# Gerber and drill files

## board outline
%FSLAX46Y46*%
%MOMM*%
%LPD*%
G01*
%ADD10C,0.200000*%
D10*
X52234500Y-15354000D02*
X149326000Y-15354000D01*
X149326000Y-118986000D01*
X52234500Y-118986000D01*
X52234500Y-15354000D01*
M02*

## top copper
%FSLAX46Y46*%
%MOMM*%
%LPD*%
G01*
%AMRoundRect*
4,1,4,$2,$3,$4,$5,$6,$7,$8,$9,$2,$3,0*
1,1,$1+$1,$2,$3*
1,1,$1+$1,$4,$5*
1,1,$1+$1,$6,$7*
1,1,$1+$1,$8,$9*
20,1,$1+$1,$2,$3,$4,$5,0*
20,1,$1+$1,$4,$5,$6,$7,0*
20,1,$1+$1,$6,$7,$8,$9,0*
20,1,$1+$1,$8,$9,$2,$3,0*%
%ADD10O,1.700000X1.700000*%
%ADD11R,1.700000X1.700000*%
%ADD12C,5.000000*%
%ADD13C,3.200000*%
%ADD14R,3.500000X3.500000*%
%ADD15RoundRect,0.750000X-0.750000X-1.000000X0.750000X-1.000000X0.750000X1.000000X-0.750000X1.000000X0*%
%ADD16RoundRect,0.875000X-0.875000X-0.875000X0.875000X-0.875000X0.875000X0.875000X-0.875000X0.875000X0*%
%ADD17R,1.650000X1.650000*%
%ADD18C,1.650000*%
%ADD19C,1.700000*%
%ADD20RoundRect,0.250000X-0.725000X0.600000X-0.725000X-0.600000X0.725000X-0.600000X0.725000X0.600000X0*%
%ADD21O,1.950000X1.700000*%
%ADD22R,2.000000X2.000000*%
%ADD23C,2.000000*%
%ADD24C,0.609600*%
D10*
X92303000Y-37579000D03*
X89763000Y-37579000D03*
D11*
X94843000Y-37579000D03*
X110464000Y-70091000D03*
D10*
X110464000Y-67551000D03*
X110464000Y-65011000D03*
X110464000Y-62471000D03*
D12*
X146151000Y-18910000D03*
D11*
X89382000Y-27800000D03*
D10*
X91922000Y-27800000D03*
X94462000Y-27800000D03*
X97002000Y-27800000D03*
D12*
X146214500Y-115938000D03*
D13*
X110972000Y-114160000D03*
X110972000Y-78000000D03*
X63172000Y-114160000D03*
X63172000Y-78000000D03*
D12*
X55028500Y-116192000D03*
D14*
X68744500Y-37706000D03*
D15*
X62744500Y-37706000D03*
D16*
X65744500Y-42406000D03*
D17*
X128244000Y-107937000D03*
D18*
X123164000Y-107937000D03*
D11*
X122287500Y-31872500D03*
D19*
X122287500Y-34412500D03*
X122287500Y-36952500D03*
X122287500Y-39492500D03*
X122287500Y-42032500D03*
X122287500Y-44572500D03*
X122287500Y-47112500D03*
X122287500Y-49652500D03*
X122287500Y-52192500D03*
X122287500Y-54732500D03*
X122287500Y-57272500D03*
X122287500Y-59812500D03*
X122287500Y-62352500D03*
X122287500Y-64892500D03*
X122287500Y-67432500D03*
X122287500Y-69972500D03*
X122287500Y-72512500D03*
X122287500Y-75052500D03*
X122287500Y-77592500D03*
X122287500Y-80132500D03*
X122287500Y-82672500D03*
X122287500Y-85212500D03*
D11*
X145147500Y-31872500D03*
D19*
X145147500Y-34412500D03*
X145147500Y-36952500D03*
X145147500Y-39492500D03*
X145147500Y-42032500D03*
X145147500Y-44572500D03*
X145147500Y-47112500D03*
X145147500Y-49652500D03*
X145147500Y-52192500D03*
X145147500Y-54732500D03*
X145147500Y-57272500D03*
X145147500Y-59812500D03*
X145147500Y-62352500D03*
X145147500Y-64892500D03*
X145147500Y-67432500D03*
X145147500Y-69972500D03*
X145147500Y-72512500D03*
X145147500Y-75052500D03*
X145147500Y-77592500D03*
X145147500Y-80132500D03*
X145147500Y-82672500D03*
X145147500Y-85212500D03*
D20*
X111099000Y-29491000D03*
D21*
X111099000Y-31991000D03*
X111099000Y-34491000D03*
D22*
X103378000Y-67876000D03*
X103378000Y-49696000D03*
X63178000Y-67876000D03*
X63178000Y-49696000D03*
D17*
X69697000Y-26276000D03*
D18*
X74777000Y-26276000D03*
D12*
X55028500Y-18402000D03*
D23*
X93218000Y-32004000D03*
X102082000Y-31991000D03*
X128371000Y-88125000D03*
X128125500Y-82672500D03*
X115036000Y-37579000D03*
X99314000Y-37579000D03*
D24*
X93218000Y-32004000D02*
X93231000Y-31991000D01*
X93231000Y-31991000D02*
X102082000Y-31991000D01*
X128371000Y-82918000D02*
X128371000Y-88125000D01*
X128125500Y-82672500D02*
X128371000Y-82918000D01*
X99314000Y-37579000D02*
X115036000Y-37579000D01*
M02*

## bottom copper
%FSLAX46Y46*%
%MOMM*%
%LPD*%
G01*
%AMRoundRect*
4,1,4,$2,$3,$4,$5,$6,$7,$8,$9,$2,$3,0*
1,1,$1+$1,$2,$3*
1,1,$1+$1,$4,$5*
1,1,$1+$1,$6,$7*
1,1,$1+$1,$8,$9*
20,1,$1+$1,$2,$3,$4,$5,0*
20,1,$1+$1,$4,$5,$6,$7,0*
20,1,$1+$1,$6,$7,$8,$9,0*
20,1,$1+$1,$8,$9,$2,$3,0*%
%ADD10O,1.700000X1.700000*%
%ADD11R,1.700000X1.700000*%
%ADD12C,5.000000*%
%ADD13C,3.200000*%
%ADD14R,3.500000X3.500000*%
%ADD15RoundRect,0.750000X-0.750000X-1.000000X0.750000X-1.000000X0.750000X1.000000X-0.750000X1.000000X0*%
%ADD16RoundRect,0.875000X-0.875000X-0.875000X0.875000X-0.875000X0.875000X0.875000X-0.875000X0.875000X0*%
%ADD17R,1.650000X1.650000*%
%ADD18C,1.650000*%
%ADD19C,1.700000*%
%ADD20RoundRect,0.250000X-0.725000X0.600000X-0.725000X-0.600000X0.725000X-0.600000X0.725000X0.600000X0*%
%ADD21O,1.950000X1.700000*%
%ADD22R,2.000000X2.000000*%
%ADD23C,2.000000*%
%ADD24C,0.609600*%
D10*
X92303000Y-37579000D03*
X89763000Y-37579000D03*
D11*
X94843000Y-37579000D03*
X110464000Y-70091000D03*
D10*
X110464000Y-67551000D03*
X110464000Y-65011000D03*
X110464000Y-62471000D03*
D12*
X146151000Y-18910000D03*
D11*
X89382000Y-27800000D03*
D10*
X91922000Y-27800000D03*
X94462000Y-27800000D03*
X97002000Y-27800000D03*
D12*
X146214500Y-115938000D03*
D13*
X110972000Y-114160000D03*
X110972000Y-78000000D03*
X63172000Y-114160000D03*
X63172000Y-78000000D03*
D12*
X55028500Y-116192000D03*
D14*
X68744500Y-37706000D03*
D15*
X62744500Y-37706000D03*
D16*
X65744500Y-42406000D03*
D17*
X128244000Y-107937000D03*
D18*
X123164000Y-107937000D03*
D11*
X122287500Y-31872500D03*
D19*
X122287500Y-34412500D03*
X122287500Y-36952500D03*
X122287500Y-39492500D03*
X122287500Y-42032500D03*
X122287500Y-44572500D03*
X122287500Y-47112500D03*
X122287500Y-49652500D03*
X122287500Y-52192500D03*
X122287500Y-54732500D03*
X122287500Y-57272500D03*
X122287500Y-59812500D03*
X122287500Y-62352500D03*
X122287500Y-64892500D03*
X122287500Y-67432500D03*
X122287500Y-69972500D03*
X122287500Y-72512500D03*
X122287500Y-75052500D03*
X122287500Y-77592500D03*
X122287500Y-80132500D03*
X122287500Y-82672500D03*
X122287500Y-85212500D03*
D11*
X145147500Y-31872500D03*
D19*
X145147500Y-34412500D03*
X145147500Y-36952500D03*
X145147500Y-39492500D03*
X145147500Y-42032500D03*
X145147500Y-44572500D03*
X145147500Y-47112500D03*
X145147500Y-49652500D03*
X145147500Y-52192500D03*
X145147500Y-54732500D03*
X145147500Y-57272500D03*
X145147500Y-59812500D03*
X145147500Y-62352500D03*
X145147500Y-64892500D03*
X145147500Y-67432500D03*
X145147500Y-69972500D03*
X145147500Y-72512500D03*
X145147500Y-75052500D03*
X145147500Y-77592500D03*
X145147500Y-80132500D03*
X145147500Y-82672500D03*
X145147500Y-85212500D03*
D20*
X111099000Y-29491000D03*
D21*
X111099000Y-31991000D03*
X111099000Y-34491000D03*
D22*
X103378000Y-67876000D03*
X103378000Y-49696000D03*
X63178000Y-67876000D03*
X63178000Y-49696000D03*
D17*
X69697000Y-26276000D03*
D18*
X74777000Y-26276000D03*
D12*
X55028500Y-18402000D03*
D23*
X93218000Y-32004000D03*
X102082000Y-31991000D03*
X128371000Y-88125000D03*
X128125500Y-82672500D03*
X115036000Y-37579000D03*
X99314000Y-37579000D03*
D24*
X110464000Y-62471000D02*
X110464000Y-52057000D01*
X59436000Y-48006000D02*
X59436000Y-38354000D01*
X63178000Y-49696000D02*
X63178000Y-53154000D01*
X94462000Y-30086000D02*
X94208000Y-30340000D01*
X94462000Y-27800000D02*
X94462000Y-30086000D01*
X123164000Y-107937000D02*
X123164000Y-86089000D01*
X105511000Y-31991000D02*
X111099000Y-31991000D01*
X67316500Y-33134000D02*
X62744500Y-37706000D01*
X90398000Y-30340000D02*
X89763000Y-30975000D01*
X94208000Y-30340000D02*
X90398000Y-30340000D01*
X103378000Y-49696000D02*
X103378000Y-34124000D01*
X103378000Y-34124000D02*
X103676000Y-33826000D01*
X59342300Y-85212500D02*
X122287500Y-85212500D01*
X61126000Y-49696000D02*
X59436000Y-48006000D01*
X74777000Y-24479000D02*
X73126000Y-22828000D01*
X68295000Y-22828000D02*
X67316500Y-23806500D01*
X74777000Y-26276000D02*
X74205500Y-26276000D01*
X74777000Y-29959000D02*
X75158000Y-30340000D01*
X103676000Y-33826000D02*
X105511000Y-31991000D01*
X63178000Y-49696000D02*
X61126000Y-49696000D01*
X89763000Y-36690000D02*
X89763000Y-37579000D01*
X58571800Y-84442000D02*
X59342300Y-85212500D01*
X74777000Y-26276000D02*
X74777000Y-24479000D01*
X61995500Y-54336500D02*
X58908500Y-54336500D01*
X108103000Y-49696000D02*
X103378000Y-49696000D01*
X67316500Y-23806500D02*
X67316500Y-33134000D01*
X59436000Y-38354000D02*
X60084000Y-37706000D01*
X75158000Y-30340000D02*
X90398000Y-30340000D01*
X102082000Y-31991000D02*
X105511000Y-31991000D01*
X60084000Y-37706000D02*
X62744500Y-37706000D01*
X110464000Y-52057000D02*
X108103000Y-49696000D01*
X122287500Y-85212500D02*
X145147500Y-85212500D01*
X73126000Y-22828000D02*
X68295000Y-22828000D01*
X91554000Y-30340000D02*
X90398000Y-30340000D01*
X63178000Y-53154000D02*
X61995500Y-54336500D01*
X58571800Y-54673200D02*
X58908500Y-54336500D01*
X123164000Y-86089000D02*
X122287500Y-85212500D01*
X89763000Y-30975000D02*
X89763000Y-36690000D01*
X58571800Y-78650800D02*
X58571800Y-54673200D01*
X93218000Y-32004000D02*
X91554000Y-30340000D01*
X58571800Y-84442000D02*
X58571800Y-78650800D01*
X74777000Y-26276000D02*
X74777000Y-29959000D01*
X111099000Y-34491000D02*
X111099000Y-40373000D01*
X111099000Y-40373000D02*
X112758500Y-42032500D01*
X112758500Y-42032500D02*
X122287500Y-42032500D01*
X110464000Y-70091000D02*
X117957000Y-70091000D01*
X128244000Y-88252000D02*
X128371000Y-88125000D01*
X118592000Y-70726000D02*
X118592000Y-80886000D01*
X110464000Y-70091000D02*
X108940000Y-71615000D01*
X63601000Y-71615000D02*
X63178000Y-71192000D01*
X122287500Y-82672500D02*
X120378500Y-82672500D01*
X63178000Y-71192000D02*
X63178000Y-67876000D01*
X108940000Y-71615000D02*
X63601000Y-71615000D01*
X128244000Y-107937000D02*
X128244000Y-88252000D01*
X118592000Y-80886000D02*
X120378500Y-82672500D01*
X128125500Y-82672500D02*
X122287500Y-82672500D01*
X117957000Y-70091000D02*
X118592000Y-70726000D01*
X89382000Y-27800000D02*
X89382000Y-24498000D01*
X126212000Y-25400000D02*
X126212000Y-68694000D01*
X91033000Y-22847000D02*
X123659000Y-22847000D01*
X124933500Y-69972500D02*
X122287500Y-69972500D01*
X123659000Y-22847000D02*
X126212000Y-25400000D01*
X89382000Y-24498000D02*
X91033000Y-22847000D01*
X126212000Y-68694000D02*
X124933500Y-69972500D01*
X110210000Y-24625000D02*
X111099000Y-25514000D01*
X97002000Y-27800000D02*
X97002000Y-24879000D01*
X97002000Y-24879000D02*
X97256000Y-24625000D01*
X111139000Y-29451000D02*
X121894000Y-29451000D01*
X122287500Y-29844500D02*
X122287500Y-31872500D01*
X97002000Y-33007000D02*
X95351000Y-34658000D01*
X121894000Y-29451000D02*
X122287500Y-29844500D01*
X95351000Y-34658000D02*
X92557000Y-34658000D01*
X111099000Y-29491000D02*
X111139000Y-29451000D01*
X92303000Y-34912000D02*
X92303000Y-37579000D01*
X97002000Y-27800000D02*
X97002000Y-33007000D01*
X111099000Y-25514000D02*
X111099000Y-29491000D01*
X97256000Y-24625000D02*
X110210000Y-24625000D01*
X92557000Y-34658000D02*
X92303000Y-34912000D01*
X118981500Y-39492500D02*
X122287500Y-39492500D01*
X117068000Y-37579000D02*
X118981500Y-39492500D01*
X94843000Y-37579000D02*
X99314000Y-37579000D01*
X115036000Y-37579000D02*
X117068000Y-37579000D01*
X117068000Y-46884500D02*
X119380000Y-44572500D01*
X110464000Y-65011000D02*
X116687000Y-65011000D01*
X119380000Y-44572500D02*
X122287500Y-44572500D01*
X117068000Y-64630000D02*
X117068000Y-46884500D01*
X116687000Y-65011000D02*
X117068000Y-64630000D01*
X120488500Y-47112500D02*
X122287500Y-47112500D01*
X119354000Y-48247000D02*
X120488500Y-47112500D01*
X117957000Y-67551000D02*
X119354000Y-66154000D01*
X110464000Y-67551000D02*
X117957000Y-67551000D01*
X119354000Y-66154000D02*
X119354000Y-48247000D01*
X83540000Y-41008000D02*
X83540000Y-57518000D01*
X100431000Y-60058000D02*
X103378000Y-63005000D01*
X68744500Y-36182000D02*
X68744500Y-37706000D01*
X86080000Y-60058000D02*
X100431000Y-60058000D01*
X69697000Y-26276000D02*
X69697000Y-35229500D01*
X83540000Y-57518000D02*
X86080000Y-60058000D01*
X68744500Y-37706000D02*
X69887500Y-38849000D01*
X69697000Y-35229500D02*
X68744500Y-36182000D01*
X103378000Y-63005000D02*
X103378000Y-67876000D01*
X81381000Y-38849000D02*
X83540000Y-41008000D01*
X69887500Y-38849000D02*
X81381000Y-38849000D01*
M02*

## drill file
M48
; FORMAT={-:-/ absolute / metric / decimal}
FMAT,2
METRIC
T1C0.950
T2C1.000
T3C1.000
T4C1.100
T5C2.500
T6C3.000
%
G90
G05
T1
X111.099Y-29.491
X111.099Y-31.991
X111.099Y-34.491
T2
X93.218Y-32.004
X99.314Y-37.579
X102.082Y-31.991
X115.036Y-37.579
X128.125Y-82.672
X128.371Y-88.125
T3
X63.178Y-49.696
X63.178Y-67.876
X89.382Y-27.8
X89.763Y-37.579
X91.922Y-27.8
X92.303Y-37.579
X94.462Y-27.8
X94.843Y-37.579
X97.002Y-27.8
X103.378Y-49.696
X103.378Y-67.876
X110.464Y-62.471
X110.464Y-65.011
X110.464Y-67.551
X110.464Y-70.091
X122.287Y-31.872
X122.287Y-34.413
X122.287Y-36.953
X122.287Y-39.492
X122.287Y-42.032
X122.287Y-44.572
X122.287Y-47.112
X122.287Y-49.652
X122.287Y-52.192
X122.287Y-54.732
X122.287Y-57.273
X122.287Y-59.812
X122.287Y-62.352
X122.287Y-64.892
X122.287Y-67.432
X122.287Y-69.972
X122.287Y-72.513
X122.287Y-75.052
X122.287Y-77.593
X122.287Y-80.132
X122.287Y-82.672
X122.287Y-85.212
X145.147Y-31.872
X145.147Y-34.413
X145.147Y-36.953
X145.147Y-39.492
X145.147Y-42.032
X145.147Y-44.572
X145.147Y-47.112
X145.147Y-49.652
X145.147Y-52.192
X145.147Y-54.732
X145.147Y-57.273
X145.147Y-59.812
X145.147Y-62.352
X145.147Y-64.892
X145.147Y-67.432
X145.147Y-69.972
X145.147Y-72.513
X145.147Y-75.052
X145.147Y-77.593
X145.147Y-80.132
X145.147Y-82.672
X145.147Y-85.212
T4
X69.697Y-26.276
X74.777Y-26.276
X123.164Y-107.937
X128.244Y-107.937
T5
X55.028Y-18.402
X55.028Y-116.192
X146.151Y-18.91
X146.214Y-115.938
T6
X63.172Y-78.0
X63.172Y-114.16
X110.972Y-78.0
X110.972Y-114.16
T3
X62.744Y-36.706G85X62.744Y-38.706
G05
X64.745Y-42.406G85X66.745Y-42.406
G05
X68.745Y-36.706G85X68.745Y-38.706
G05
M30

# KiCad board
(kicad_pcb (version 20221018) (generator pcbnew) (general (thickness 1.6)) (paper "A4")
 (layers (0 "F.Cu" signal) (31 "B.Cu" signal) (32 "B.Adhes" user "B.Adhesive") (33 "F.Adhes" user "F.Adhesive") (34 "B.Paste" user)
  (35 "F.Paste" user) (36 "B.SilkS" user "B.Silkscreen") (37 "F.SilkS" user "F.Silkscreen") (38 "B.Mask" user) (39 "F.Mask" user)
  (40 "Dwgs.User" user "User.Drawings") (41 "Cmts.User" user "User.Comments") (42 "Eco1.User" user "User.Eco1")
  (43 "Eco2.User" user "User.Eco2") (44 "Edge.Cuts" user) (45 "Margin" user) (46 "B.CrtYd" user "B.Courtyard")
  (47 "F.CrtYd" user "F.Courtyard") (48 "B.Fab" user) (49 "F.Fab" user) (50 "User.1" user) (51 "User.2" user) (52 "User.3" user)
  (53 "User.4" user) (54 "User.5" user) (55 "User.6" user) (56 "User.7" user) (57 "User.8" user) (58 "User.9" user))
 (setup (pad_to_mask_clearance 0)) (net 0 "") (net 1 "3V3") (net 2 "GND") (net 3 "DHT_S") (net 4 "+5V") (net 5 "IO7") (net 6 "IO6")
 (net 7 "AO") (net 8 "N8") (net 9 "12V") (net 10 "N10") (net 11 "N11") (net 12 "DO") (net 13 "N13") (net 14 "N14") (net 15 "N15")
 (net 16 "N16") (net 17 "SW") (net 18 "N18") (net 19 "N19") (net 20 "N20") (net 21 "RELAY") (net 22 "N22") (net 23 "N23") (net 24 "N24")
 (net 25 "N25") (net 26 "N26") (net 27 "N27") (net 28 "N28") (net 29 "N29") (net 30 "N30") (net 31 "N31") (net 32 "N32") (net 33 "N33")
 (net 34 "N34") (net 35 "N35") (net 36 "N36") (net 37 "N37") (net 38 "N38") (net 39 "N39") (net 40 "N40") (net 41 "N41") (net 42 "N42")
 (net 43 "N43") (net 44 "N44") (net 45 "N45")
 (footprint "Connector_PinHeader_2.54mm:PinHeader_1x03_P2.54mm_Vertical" (layer "F.Cu") (at 94.843 37.579 -90)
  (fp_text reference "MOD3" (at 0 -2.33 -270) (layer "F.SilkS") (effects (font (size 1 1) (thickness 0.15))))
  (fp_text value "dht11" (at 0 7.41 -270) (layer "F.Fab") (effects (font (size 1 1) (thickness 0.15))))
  (pad "+" thru_hole oval (at 0 2.54 270) (size 1.7 1.7) (drill 1) (layers "*.Cu" "*.Mask") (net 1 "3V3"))
  (pad "-" thru_hole oval (at 0 5.08 270) (size 1.7 1.7) (drill 1) (layers "*.Cu" "*.Mask") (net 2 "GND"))
  (pad "S" thru_hole rect (at 0 0 270) (size 1.7 1.7) (drill 1) (layers "*.Cu" "*.Mask") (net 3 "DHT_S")))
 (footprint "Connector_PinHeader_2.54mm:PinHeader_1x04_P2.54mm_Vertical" (layer "F.Cu") (at 110.464 70.091 180)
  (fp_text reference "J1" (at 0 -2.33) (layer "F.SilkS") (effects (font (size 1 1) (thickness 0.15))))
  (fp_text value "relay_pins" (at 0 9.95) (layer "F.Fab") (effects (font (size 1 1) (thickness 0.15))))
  (pad "1" thru_hole rect (at 0 0 180) (size 1.7 1.7) (drill 1) (layers "*.Cu" "*.Mask") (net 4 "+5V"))
  (pad "2" thru_hole oval (at 0 2.54 180) (size 1.7 1.7) (drill 1) (layers "*.Cu" "*.Mask") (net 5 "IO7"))
  (pad "3" thru_hole oval (at 0 5.08 180) (size 1.7 1.7) (drill 1) (layers "*.Cu" "*.Mask") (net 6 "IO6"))
  (pad "4" thru_hole oval (at 0 7.62 180) (size 1.7 1.7) (drill 1) (layers "*.Cu" "*.Mask") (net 2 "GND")))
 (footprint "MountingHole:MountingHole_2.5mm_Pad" (layer "F.Cu") (at 146.151 18.91)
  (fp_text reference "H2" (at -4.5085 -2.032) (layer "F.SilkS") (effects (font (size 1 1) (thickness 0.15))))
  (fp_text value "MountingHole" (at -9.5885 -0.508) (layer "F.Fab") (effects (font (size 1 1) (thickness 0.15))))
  (pad "1" thru_hole circle (at 0 0) (size 5 5) (drill 2.5) (layers "*.Cu" "*.Mask")))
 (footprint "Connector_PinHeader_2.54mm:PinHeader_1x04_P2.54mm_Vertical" (layer "F.Cu") (at 89.382 27.8 90)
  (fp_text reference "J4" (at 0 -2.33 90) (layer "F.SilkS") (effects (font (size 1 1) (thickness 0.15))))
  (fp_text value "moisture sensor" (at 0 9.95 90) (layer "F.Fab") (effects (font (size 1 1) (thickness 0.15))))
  (pad "1" thru_hole rect (at 0 0 90) (size 1.7 1.7) (drill 1) (layers "*.Cu" "*.Mask") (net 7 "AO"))
  (pad "2" thru_hole oval (at 0 2.54 90) (size 1.7 1.7) (drill 1) (layers "*.Cu" "*.Mask") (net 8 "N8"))
  (pad "3" thru_hole oval (at 0 5.08 90) (size 1.7 1.7) (drill 1) (layers "*.Cu" "*.Mask") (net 2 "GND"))
  (pad "4" thru_hole oval (at 0 7.62 90) (size 1.7 1.7) (drill 1) (layers "*.Cu" "*.Mask") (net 1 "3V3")))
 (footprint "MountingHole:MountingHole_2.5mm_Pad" (layer "F.Cu") (at 146.2145 115.938)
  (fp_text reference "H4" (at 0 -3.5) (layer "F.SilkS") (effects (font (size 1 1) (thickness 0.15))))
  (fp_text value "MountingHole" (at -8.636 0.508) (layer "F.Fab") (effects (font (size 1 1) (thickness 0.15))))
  (pad "1" thru_hole circle (at 0 0) (size 5 5) (drill 2.5) (layers "*.Cu" "*.Mask")))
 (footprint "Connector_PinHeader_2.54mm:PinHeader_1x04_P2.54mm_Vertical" (layer "F.Cu") (at 110.972 114.16 180)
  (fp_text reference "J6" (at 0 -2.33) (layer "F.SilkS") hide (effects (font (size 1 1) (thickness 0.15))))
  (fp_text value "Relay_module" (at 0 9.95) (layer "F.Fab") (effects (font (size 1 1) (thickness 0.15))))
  (pad "" np_thru_hole circle (at 0 0 180) (size 3.2 3.2) (drill 3) (layers "F&B.Cu" "*.Mask"))
  (pad "" np_thru_hole circle (at 0 36.16 180) (size 3.2 3.2) (drill 3) (layers "F&B.Cu" "*.Mask"))
  (pad "" np_thru_hole circle (at 47.8 0 180) (size 3.2 3.2) (drill 3) (layers "F&B.Cu" "*.Mask"))
  (pad "" np_thru_hole circle (at 47.8 36.16 180) (size 3.2 3.2) (drill 3) (layers "F&B.Cu" "*.Mask")))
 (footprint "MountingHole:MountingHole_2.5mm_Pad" (layer "F.Cu") (at 55.0285 116.192)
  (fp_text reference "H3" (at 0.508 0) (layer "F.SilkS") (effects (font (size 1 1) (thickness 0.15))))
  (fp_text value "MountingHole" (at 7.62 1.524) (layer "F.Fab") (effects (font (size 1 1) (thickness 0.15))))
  (pad "1" thru_hole circle (at 0 0) (size 5 5) (drill 2.5) (layers "*.Cu" "*.Mask")))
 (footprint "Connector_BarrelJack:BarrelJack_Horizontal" (layer "F.Cu") (at 68.7445 37.706)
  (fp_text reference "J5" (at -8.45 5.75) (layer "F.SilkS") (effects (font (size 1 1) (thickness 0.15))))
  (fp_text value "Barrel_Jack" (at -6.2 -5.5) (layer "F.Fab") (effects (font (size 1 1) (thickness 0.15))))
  (pad "1" thru_hole rect (at 0 0) (size 3.5 3.5) (drill oval 1 3) (layers "*.Cu" "*.Mask") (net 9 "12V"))
  (pad "2" thru_hole roundrect (at -6 0) (size 3 3.5) (drill oval 1 3) (layers "*.Cu" "*.Mask") (roundrect_rratio 0.25) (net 2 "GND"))
  (pad "3" thru_hole roundrect (at -3 4.7) (size 3.5 3.5) (drill oval 3 1) (layers "*.Cu" "*.Mask") (roundrect_rratio 0.25)))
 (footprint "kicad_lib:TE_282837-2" (layer "F.Cu") (at 125.704 107.937 180)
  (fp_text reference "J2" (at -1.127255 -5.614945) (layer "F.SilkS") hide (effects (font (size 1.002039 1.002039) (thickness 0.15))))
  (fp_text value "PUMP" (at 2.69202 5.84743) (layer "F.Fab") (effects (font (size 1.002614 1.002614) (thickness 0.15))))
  (pad "1" thru_hole rect (at -2.54 0 180) (size 1.65 1.65) (drill 1.1) (layers "*.Cu" "*.Mask") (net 4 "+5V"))
  (pad "2" thru_hole circle (at 2.54 0 180) (size 1.65 1.65) (drill 1.1) (layers "*.Cu" "*.Mask") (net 2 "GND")))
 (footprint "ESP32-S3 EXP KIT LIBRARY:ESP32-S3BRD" (layer "F.Cu") (at 121.0175 96.6725)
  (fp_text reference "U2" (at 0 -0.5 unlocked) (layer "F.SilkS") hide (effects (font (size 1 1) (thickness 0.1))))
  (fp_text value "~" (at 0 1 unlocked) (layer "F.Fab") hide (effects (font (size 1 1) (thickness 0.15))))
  (pad "1_1" thru_hole rect (at 1.27 -64.8) (size 1.7 1.7) (drill 1) (layers "*.Cu" "*.Mask") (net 1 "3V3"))
  (pad "1_2" thru_hole circle (at 1.27 -62.26) (size 1.7 1.7) (drill 1) (layers "*.Cu" "*.Mask") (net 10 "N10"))
  (pad "1_3" thru_hole circle (at 1.27 -59.72) (size 1.7 1.7) (drill 1) (layers "*.Cu" "*.Mask") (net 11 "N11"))
  (pad "1_4" thru_hole circle (at 1.27 -57.18) (size 1.7 1.7) (drill 1) (layers "*.Cu" "*.Mask") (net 3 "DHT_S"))
  (pad "1_5" thru_hole circle (at 1.27 -54.64) (size 1.7 1.7) (drill 1) (layers "*.Cu" "*.Mask") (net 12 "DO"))
  (pad "1_6" thru_hole circle (at 1.27 -52.1) (size 1.7 1.7) (drill 1) (layers "*.Cu" "*.Mask") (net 6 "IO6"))
  (pad "1_7" thru_hole circle (at 1.27 -49.56) (size 1.7 1.7) (drill 1) (layers "*.Cu" "*.Mask") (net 5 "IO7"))
  (pad "1_8" thru_hole circle (at 1.27 -47.02) (size 1.7 1.7) (drill 1) (layers "*.Cu" "*.Mask") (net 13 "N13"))
  (pad "1_9" thru_hole circle (at 1.27 -44.48) (size 1.7 1.7) (drill 1) (layers "*.Cu" "*.Mask") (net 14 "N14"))
  (pad "1_10" thru_hole circle (at 1.27 -41.94) (size 1.7 1.7) (drill 1) (layers "*.Cu" "*.Mask") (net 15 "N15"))
  (pad "1_11" thru_hole circle (at 1.27 -39.4) (size 1.7 1.7) (drill 1) (layers "*.Cu" "*.Mask") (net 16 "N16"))
  (pad "1_12" thru_hole circle (at 1.27 -36.86) (size 1.7 1.7) (drill 1) (layers "*.Cu" "*.Mask") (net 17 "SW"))
  (pad "1_13" thru_hole circle (at 1.27 -34.32) (size 1.7 1.7) (drill 1) (layers "*.Cu" "*.Mask") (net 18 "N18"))
  (pad "1_14" thru_hole circle (at 1.27 -31.78) (size 1.7 1.7) (drill 1) (layers "*.Cu" "*.Mask") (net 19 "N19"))
  (pad "1_15" thru_hole circle (at 1.27 -29.24) (size 1.7 1.7) (drill 1) (layers "*.Cu" "*.Mask") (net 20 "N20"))
  (pad "1_16" thru_hole circle (at 1.27 -26.7) (size 1.7 1.7) (drill 1) (layers "*.Cu" "*.Mask") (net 7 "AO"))
  (pad "1_17" thru_hole circle (at 1.27 -24.16) (size 1.7 1.7) (drill 1) (layers "*.Cu" "*.Mask") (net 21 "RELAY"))
  (pad "1_18" thru_hole circle (at 1.27 -21.62) (size 1.7 1.7) (drill 1) (layers "*.Cu" "*.Mask") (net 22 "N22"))
  (pad "1_19" thru_hole circle (at 1.27 -19.08) (size 1.7 1.7) (drill 1) (layers "*.Cu" "*.Mask") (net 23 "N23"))
  (pad "1_20" thru_hole circle (at 1.27 -16.54) (size 1.7 1.7) (drill 1) (layers "*.Cu" "*.Mask") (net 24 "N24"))
  (pad "1_21" thru_hole circle (at 1.27 -14) (size 1.7 1.7) (drill 1) (layers "*.Cu" "*.Mask") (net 4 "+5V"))
  (pad "1_22" thru_hole circle (at 1.27 -11.46) (size 1.7 1.7) (drill 1) (layers "*.Cu" "*.Mask") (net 2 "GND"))
  (pad "2_1" thru_hole rect (at 24.13 -64.8) (size 1.7 1.7) (drill 1) (layers "*.Cu" "*.Mask") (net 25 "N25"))
  (pad "2_2" thru_hole circle (at 24.13 -62.26) (size 1.7 1.7) (drill 1) (layers "*.Cu" "*.Mask") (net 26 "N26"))
  (pad "2_3" thru_hole circle (at 24.13 -59.72) (size 1.7 1.7) (drill 1) (layers "*.Cu" "*.Mask") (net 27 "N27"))
  (pad "2_4" thru_hole circle (at 24.13 -57.18) (size 1.7 1.7) (drill 1) (layers "*.Cu" "*.Mask") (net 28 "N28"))
  (pad "2_5" thru_hole circle (at 24.13 -54.64) (size 1.7 1.7) (drill 1) (layers "*.Cu" "*.Mask") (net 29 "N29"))
  (pad "2_6" thru_hole circle (at 24.13 -52.1) (size 1.7 1.7) (drill 1) (layers "*.Cu" "*.Mask") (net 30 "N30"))
  (pad "2_7" thru_hole circle (at 24.13 -49.56) (size 1.7 1.7) (drill 1) (layers "*.Cu" "*.Mask") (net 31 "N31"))
  (pad "2_8" thru_hole circle (at 24.13 -47.02) (size 1.7 1.7) (drill 1) (layers "*.Cu" "*.Mask") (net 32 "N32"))
  (pad "2_9" thru_hole circle (at 24.13 -44.48) (size 1.7 1.7) (drill 1) (layers "*.Cu" "*.Mask") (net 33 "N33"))
  (pad "2_10" thru_hole circle (at 24.13 -41.94) (size 1.7 1.7) (drill 1) (layers "*.Cu" "*.Mask") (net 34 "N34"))
  (pad "2_11" thru_hole circle (at 24.13 -39.4) (size 1.7 1.7) (drill 1) (layers "*.Cu" "*.Mask") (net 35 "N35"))
  (pad "2_12" thru_hole circle (at 24.13 -36.86) (size 1.7 1.7) (drill 1) (layers "*.Cu" "*.Mask") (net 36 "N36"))
  (pad "2_13" thru_hole circle (at 24.13 -34.32) (size 1.7 1.7) (drill 1) (layers "*.Cu" "*.Mask") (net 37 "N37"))
  (pad "2_14" thru_hole circle (at 24.13 -31.78) (size 1.7 1.7) (drill 1) (layers "*.Cu" "*.Mask") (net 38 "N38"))
  (pad "2_15" thru_hole circle (at 24.13 -29.24) (size 1.7 1.7) (drill 1) (layers "*.Cu" "*.Mask") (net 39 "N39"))
  (pad "2_16" thru_hole circle (at 24.13 -26.7) (size 1.7 1.7) (drill 1) (layers "*.Cu" "*.Mask") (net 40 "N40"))
  (pad "2_17" thru_hole circle (at 24.13 -24.16) (size 1.7 1.7) (drill 1) (layers "*.Cu" "*.Mask") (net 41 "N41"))
  (pad "2_18" thru_hole circle (at 24.13 -21.62) (size 1.7 1.7) (drill 1) (layers "*.Cu" "*.Mask") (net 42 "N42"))
  (pad "2_19" thru_hole circle (at 24.13 -19.08) (size 1.7 1.7) (drill 1) (layers "*.Cu" "*.Mask") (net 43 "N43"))
  (pad "2_20" thru_hole circle (at 24.13 -16.54) (size 1.7 1.7) (drill 1) (layers "*.Cu" "*.Mask") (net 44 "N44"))
  (pad "2_21" thru_hole circle (at 24.13 -14) (size 1.7 1.7) (drill 1) (layers "*.Cu" "*.Mask") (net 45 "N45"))
  (pad "2_22" thru_hole circle (at 24.13 -11.46) (size 1.7 1.7) (drill 1) (layers "*.Cu" "*.Mask") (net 2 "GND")))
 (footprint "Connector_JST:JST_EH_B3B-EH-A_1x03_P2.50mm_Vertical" (layer "F.Cu") (at 111.099 29.491 -90)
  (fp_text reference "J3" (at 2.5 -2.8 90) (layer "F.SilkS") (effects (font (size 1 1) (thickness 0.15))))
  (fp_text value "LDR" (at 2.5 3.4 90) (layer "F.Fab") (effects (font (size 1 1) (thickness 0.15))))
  (pad "1" thru_hole roundrect (at 0 0 270) (size 1.7 1.95) (drill 0.95) (layers "*.Cu" "*.Mask") (roundrect_rratio 0.147059) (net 1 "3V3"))
  (pad "2" thru_hole oval (at 2.5 0 270) (size 1.7 1.95) (drill 0.95) (layers "*.Cu" "*.Mask") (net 2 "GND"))
  (pad "3" thru_hole oval (at 5 0 270) (size 1.7 1.95) (drill 0.95) (layers "*.Cu" "*.Mask") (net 12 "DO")))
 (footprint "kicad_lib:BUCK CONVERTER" (layer "F.Cu") (at 105.178 47.896 180)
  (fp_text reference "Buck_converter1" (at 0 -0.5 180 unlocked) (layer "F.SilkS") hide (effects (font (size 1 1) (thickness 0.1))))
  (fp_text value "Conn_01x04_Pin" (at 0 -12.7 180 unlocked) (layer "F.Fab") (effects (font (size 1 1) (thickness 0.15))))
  (pad "IN+" thru_hole rect (at 1.8 -19.98 180) (size 2 2) (drill 1) (layers "*.Cu" "*.Mask") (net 9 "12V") (thermal_bridge_angle 45))
  (pad "IN-" thru_hole rect (at 1.8 -1.8 180) (size 2 2) (drill 1) (layers "*.Cu" "B.Mask") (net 2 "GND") (thermal_bridge_angle 45))
  (pad "OUT+" thru_hole rect (at 42 -19.98 180) (size 2 2) (drill 1) (layers "*.Cu" "*.Mask") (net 4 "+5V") (thermal_bridge_angle 45))
  (pad "OUT-" thru_hole rect (at 42 -1.8 180) (size 2 2) (drill 1) (layers "*.Cu" "*.Mask") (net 2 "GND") (thermal_bridge_angle 45)))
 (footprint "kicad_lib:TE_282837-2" (layer "F.Cu") (at 72.237 26.276)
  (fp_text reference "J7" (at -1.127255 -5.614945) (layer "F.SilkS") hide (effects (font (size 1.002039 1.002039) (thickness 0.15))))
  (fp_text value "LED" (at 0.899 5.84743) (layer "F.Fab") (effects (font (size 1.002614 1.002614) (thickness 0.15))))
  (pad "1" thru_hole rect (at -2.54 0) (size 1.65 1.65) (drill 1.1) (layers "*.Cu" "*.Mask") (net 9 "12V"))
  (pad "2" thru_hole circle (at 2.54 0) (size 1.65 1.65) (drill 1.1) (layers "*.Cu" "*.Mask") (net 2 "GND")))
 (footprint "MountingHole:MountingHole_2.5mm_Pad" (layer "F.Cu") (at 55.0285 18.402)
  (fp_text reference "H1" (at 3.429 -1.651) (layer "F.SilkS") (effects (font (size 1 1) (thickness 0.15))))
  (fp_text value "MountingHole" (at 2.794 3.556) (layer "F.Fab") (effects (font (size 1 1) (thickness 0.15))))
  (pad "1" thru_hole circle (at 0 0) (size 5 5) (drill 2.5) (layers "*.Cu" "*.Mask")))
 (gr_rect (start 52.2345 15.354) (end 149.326 118.986) (stroke (width 0.2) (type default)) (fill none) (layer "Edge.Cuts"))
 (segment (start 93.218 32.004) (end 93.231 31.991) (width 0.6096) (layer "F.Cu") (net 2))
 (segment (start 93.231 31.991) (end 102.082 31.991) (width 0.6096) (layer "F.Cu") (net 2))
 (via (at 93.218 32.004) (size 2) (drill 1) (layers "F.Cu" "B.Cu") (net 2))
 (via (at 102.082 31.991) (size 2) (drill 1) (layers "F.Cu" "B.Cu") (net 2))
 (segment (start 110.464 62.471) (end 110.464 52.057) (width 0.6096) (layer "B.Cu") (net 2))
 (segment (start 59.436 48.006) (end 59.436 38.354) (width 0.6096) (layer "B.Cu") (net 2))
 (segment (start 63.178 49.696) (end 63.178 53.154) (width 0.6096) (layer "B.Cu") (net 2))
 (segment (start 94.462 30.086) (end 94.208 30.34) (width 0.6096) (layer "B.Cu") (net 2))
 (segment (start 94.462 27.8) (end 94.462 30.086) (width 0.6096) (layer "B.Cu") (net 2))
 (segment (start 123.164 107.937) (end 123.164 86.089) (width 0.6096) (layer "B.Cu") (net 2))
 (segment (start 105.511 31.991) (end 111.099 31.991) (width 0.6096) (layer "B.Cu") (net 2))
 (segment (start 67.3165 33.134) (end 62.7445 37.706) (width 0.6096) (layer "B.Cu") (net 2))
 (segment (start 90.398 30.34) (end 89.763 30.975) (width 0.6096) (layer "B.Cu") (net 2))
 (segment (start 94.208 30.34) (end 90.398 30.34) (width 0.6096) (layer "B.Cu") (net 2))
 (segment (start 103.378 49.696) (end 103.378 34.124) (width 0.6096) (layer "B.Cu") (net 2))
 (segment (start 103.378 34.124) (end 103.676 33.826) (width 0.6096) (layer "B.Cu") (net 2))
 (segment (start 59.3423 85.2125) (end 122.2875 85.2125) (width 0.6096) (layer "B.Cu") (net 2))
 (segment (start 61.126 49.696) (end 59.436 48.006) (width 0.6096) (layer "B.Cu") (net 2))
 (segment (start 74.777 24.479) (end 73.126 22.828) (width 0.6096) (layer "B.Cu") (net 2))
 (segment (start 68.295 22.828) (end 67.3165 23.8065) (width 0.6096) (layer "B.Cu") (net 2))
 (segment (start 74.777 26.276) (end 74.2055 26.276) (width 0.6096) (layer "B.Cu") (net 2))
 (segment (start 74.777 29.959) (end 75.158 30.34) (width 0.6096) (layer "B.Cu") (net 2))
 (segment (start 103.676 33.826) (end 105.511 31.991) (width 0.6096) (layer "B.Cu") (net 2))
 (segment (start 63.178 49.696) (end 61.126 49.696) (width 0.6096) (layer "B.Cu") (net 2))
 (segment (start 89.763 36.69) (end 89.763 37.579) (width 0.6096) (layer "B.Cu") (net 2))
 (segment (start 58.5718 84.442) (end 59.3423 85.2125) (width 0.6096) (layer "B.Cu") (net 2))
 (segment (start 74.777 26.276) (end 74.777 24.479) (width 0.6096) (layer "B.Cu") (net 2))
 (segment (start 61.9955 54.3365) (end 58.9085 54.3365) (width 0.6096) (layer "B.Cu") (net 2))
 (segment (start 108.103 49.696) (end 103.378 49.696) (width 0.6096) (layer "B.Cu") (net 2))
 (segment (start 67.3165 23.8065) (end 67.3165 33.134) (width 0.6096) (layer "B.Cu") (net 2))
 (segment (start 59.436 38.354) (end 60.084 37.706) (width 0.6096) (layer "B.Cu") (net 2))
 (segment (start 75.158 30.34) (end 90.398 30.34) (width 0.6096) (layer "B.Cu") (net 2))
 (segment (start 102.082 31.991) (end 105.511 31.991) (width 0.6096) (layer "B.Cu") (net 2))
 (segment (start 60.084 37.706) (end 62.7445 37.706) (width 0.6096) (layer "B.Cu") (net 2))
 (segment (start 110.464 52.057) (end 108.103 49.696) (width 0.6096) (layer "B.Cu") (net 2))
 (segment (start 122.2875 85.2125) (end 145.1475 85.2125) (width 0.6096) (layer "B.Cu") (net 2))
 (segment (start 73.126 22.828) (end 68.295 22.828) (width 0.6096) (layer "B.Cu") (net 2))
 (segment (start 91.554 30.34) (end 90.398 30.34) (width 0.6096) (layer "B.Cu") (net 2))
 (segment (start 63.178 53.154) (end 61.9955 54.3365) (width 0.6096) (layer "B.Cu") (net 2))
 (segment (start 58.5718 54.6732) (end 58.9085 54.3365) (width 0.6096) (layer "B.Cu") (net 2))
 (segment (start 123.164 86.089) (end 122.2875 85.2125) (width 0.6096) (layer "B.Cu") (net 2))
 (segment (start 89.763 30.975) (end 89.763 36.69) (width 0.6096) (layer "B.Cu") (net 2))
 (segment (start 58.5718 78.6508) (end 58.5718 54.6732) (width 0.6096) (layer "B.Cu") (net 2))
 (segment (start 93.218 32.004) (end 91.554 30.34) (width 0.6096) (layer "B.Cu") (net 2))
 (segment (start 58.5718 84.442) (end 58.5718 78.6508) (width 0.6096) (layer "B.Cu") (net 2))
 (segment (start 74.777 26.276) (end 74.777 29.959) (width 0.6096) (layer "B.Cu") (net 2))
 (segment (start 111.099 34.491) (end 111.099 40.373) (width 0.6096) (layer "B.Cu") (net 12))
 (segment (start 111.099 40.373) (end 112.7585 42.0325) (width 0.6096) (layer "B.Cu") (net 12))
 (segment (start 112.7585 42.0325) (end 122.2875 42.0325) (width 0.6096) (layer "B.Cu") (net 12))
 (segment (start 128.371 82.918) (end 128.371 88.125) (width 0.6096) (layer "F.Cu") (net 4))
 (segment (start 128.1255 82.6725) (end 128.371 82.918) (width 0.6096) (layer "F.Cu") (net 4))
 (via (at 128.371 88.125) (size 2) (drill 1) (layers "F.Cu" "B.Cu") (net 4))
 (via (at 128.1255 82.6725) (size 2) (drill 1) (layers "F.Cu" "B.Cu") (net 4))
 (segment (start 110.464 70.091) (end 117.957 70.091) (width 0.6096) (layer "B.Cu") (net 4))
 (segment (start 128.244 88.252) (end 128.371 88.125) (width 0.6096) (layer "B.Cu") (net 4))
 (segment (start 118.592 70.726) (end 118.592 80.886) (width 0.6096) (layer "B.Cu") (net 4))
 (segment (start 110.464 70.091) (end 108.94 71.615) (width 0.6096) (layer "B.Cu") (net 4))
 (segment (start 63.601 71.615) (end 63.178 71.192) (width 0.6096) (layer "B.Cu") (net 4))
 (segment (start 122.2875 82.6725) (end 120.3785 82.6725) (width 0.6096) (layer "B.Cu") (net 4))
 (segment (start 63.178 71.192) (end 63.178 67.876) (width 0.6096) (layer "B.Cu") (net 4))
 (segment (start 108.94 71.615) (end 63.601 71.615) (width 0.6096) (layer "B.Cu") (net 4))
 (segment (start 128.244 107.937) (end 128.244 88.252) (width 0.6096) (layer "B.Cu") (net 4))
 (segment (start 118.592 80.886) (end 120.3785 82.6725) (width 0.6096) (layer "B.Cu") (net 4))
 (segment (start 128.1255 82.6725) (end 122.2875 82.6725) (width 0.6096) (layer "B.Cu") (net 4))
 (segment (start 117.957 70.091) (end 118.592 70.726) (width 0.6096) (layer "B.Cu") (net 4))
 (segment (start 89.382 27.8) (end 89.382 24.498) (width 0.6096) (layer "B.Cu") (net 7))
 (segment (start 126.212 25.4) (end 126.212 68.694) (width 0.6096) (layer "B.Cu") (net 7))
 (segment (start 91.033 22.847) (end 123.659 22.847) (width 0.6096) (layer "B.Cu") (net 7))
 (segment (start 124.9335 69.9725) (end 122.2875 69.9725) (width 0.6096) (layer "B.Cu") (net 7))
 (segment (start 123.659 22.847) (end 126.212 25.4) (width 0.6096) (layer "B.Cu") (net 7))
 (segment (start 89.382 24.498) (end 91.033 22.847) (width 0.6096) (layer "B.Cu") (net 7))
 (segment (start 126.212 68.694) (end 124.9335 69.9725) (width 0.6096) (layer "B.Cu") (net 7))
 (segment (start 110.21 24.625) (end 111.099 25.514) (width 0.6096) (layer "B.Cu") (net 1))
 (segment (start 97.002 27.8) (end 97.002 24.879) (width 0.6096) (layer "B.Cu") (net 1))
 (segment (start 97.002 24.879) (end 97.256 24.625) (width 0.6096) (layer "B.Cu") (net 1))
 (segment (start 111.139 29.451) (end 121.894 29.451) (width 0.6096) (layer "B.Cu") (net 1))
 (segment (start 122.2875 29.8445) (end 122.2875 31.8725) (width 0.6096) (layer "B.Cu") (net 1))
 (segment (start 97.002 33.007) (end 95.351 34.658) (width 0.6096) (layer "B.Cu") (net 1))
 (segment (start 121.894 29.451) (end 122.2875 29.8445) (width 0.6096) (layer "B.Cu") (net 1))
 (segment (start 95.351 34.658) (end 92.557 34.658) (width 0.6096) (layer "B.Cu") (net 1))
 (segment (start 111.099 29.491) (end 111.139 29.451) (width 0.6096) (layer "B.Cu") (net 1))
 (segment (start 92.303 34.912) (end 92.303 37.579) (width 0.6096) (layer "B.Cu") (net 1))
 (segment (start 97.002 27.8) (end 97.002 33.007) (width 0.6096) (layer "B.Cu") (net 1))
 (segment (start 111.099 25.514) (end 111.099 29.491) (width 0.6096) (layer "B.Cu") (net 1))
 (segment (start 97.256 24.625) (end 110.21 24.625) (width 0.6096) (layer "B.Cu") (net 1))
 (segment (start 92.557 34.658) (end 92.303 34.912) (width 0.6096) (layer "B.Cu") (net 1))
 (segment (start 99.314 37.579) (end 115.036 37.579) (width 0.6096) (layer "F.Cu") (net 3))
 (via (at 115.036 37.579) (size 2) (drill 1) (layers "F.Cu" "B.Cu") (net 3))
 (via (at 99.314 37.579) (size 2) (drill 1) (layers "F.Cu" "B.Cu") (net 3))
 (segment (start 118.9815 39.4925) (end 122.2875 39.4925) (width 0.6096) (layer "B.Cu") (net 3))
 (segment (start 117.068 37.579) (end 118.9815 39.4925) (width 0.6096) (layer "B.Cu") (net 3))
 (segment (start 94.843 37.579) (end 99.314 37.579) (width 0.6096) (layer "B.Cu") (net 3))
 (segment (start 115.036 37.579) (end 117.068 37.579) (width 0.6096) (layer "B.Cu") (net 3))
 (segment (start 117.068 46.8845) (end 119.38 44.5725) (width 0.6096) (layer "B.Cu") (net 6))
 (segment (start 110.464 65.011) (end 116.687 65.011) (width 0.6096) (layer "B.Cu") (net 6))
 (segment (start 119.38 44.5725) (end 122.2875 44.5725) (width 0.6096) (layer "B.Cu") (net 6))
 (segment (start 117.068 64.63) (end 117.068 46.8845) (width 0.6096) (layer "B.Cu") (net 6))
 (segment (start 116.687 65.011) (end 117.068 64.63) (width 0.6096) (layer "B.Cu") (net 6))
 (segment (start 120.4885 47.1125) (end 122.2875 47.1125) (width 0.6096) (layer "B.Cu") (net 5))
 (segment (start 119.354 48.247) (end 120.4885 47.1125) (width 0.6096) (layer "B.Cu") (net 5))
 (segment (start 117.957 67.551) (end 119.354 66.154) (width 0.6096) (layer "B.Cu") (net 5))
 (segment (start 110.464 67.551) (end 117.957 67.551) (width 0.6096) (layer "B.Cu") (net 5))
 (segment (start 119.354 66.154) (end 119.354 48.247) (width 0.6096) (layer "B.Cu") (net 5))
 (segment (start 83.54 41.008) (end 83.54 57.518) (width 0.6096) (layer "B.Cu") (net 9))
 (segment (start 100.431 60.058) (end 103.378 63.005) (width 0.6096) (layer "B.Cu") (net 9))
 (segment (start 68.7445 36.182) (end 68.7445 37.706) (width 0.6096) (layer "B.Cu") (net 9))
 (segment (start 86.08 60.058) (end 100.431 60.058) (width 0.6096) (layer "B.Cu") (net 9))
 (segment (start 69.697 26.276) (end 69.697 35.2295) (width 0.6096) (layer "B.Cu") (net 9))
 (segment (start 83.54 57.518) (end 86.08 60.058) (width 0.6096) (layer "B.Cu") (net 9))
 (segment (start 68.7445 37.706) (end 69.8875 38.849) (width 0.6096) (layer "B.Cu") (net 9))
 (segment (start 69.697 35.2295) (end 68.7445 36.182) (width 0.6096) (layer "B.Cu") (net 9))
 (segment (start 103.378 63.005) (end 103.378 67.876) (width 0.6096) (layer "B.Cu") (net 9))
 (segment (start 81.381 38.849) (end 83.54 41.008) (width 0.6096) (layer "B.Cu") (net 9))
 (segment (start 69.8875 38.849) (end 81.381 38.849) (width 0.6096) (layer "B.Cu") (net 9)))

